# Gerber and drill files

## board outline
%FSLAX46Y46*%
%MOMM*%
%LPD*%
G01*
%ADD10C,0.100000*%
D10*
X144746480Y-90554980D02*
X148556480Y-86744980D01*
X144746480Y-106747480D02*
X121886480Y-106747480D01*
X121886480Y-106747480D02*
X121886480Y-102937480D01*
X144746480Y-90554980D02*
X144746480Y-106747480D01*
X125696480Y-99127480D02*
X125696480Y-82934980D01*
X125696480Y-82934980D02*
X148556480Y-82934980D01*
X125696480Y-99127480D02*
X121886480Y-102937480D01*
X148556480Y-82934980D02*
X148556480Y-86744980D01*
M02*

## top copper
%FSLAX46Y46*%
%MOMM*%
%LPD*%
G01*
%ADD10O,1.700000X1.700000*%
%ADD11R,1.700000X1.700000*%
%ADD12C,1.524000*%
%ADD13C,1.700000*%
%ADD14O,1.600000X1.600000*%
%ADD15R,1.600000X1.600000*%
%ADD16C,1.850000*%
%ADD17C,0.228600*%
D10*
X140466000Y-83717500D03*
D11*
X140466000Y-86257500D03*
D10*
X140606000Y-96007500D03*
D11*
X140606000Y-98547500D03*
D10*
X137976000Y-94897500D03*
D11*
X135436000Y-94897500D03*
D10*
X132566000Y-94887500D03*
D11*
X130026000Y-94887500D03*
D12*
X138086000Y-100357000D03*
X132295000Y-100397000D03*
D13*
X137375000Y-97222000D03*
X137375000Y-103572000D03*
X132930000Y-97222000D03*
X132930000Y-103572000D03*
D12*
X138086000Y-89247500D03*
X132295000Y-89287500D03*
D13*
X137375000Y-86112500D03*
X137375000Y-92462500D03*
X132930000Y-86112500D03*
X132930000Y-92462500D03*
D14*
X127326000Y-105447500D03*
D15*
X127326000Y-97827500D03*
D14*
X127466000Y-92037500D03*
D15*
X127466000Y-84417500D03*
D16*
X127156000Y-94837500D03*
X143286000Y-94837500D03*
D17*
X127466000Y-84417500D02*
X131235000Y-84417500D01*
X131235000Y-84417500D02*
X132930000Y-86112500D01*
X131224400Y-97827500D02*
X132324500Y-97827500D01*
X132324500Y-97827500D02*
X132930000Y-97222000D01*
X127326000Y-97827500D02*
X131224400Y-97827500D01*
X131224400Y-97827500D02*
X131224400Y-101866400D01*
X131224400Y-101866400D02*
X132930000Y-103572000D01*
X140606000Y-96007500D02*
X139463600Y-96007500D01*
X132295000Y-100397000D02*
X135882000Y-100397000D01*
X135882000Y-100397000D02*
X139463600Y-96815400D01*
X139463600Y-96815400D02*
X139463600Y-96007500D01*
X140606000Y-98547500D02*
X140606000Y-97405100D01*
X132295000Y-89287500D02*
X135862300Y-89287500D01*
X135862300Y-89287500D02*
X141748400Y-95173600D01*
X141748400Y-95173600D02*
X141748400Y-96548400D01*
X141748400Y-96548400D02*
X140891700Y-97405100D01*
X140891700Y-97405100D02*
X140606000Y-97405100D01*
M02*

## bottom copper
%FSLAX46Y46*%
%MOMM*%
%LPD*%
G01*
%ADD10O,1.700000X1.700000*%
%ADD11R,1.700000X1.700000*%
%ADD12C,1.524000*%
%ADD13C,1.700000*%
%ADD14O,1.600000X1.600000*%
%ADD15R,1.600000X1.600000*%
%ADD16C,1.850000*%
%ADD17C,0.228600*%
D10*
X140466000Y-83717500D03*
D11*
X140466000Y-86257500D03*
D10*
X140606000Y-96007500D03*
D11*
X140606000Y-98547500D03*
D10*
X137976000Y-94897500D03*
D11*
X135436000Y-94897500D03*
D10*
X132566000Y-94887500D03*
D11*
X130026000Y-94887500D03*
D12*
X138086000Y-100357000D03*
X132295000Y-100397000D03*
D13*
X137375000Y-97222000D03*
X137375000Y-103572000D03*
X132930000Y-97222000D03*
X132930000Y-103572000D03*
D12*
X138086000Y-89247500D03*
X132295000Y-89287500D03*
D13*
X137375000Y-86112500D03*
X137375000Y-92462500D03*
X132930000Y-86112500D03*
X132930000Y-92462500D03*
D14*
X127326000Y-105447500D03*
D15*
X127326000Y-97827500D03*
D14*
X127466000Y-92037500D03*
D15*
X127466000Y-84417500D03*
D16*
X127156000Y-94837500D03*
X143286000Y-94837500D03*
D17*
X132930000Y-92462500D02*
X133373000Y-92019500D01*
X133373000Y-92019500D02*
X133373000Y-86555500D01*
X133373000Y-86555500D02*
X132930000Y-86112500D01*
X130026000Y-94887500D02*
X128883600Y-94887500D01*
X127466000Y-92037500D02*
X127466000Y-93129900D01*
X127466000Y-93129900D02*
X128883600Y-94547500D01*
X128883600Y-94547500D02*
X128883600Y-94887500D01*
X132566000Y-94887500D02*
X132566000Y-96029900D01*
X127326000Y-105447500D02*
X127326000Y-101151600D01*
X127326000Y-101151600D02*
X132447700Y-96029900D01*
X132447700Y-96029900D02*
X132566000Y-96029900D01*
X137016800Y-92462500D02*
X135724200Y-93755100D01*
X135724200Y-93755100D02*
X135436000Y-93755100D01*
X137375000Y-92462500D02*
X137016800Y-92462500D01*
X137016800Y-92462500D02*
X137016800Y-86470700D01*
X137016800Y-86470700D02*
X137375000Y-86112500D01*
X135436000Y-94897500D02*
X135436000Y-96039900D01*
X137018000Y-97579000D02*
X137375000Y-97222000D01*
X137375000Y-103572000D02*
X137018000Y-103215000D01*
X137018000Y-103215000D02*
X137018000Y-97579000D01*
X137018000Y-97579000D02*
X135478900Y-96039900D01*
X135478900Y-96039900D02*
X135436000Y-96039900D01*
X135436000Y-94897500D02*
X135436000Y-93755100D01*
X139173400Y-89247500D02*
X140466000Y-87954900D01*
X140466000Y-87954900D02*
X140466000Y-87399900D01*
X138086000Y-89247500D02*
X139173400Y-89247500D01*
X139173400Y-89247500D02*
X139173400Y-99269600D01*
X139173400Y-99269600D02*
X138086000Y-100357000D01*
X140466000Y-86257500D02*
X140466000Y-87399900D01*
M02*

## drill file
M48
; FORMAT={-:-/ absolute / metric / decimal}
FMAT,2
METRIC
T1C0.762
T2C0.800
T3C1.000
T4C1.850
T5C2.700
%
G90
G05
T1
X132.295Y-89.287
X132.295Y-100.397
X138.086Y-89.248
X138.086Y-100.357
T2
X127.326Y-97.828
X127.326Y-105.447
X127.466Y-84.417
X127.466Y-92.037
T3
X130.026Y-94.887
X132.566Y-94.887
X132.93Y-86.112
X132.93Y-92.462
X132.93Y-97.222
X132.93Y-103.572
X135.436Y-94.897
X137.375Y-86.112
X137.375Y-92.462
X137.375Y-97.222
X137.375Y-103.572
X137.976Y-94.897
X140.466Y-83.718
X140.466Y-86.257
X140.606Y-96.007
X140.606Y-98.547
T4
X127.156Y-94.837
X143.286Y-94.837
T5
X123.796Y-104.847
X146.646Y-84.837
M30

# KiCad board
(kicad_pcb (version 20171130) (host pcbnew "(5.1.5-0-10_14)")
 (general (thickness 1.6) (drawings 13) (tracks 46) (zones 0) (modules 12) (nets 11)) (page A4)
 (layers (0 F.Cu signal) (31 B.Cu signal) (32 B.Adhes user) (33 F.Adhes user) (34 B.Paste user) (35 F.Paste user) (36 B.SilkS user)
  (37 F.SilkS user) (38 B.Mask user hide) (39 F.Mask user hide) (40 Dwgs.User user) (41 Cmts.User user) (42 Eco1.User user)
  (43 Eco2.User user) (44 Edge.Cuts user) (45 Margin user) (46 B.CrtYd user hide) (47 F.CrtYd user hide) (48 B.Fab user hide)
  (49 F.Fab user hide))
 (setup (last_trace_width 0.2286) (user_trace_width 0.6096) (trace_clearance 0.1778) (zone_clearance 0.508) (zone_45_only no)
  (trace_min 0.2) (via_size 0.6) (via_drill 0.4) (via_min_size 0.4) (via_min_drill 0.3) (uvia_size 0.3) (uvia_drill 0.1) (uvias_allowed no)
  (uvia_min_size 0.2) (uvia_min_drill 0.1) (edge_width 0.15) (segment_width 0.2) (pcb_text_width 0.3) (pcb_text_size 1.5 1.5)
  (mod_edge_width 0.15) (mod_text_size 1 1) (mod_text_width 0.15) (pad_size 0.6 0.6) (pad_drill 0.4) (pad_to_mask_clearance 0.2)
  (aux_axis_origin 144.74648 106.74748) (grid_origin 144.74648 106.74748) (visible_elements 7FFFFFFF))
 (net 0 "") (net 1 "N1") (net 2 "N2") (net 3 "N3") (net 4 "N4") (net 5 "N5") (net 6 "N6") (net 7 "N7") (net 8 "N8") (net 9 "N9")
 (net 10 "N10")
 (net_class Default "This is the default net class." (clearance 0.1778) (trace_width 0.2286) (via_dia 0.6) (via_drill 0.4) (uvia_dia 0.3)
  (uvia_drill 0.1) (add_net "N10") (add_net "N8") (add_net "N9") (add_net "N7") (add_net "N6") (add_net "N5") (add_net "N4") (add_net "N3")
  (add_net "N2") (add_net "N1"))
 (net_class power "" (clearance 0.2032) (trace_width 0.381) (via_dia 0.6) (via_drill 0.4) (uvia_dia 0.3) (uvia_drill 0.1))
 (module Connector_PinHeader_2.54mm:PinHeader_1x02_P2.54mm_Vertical (layer B.Cu) (at 140.466 86.2575)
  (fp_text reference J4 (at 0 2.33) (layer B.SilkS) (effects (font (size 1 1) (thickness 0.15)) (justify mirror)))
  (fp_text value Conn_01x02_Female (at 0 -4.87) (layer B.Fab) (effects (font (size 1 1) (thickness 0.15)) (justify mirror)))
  (pad 2 thru_hole oval (at 0 -2.54) (size 1.7 1.7) (drill 1) (layers *.Cu *.Mask) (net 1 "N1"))
  (pad 1 thru_hole rect (at 0 0) (size 1.7 1.7) (drill 1) (layers *.Cu *.Mask) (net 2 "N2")))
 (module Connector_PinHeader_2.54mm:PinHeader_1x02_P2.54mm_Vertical (layer B.Cu) (at 140.606 98.5475)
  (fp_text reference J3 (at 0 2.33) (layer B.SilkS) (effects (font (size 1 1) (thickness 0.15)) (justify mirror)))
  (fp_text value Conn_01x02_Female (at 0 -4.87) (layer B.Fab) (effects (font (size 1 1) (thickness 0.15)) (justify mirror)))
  (pad 2 thru_hole oval (at 0 -2.54) (size 1.7 1.7) (drill 1) (layers *.Cu *.Mask) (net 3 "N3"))
  (pad 1 thru_hole rect (at 0 0) (size 1.7 1.7) (drill 1) (layers *.Cu *.Mask) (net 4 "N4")))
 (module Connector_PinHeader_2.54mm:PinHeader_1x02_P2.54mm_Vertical (layer B.Cu) (at 135.436 94.8975 270)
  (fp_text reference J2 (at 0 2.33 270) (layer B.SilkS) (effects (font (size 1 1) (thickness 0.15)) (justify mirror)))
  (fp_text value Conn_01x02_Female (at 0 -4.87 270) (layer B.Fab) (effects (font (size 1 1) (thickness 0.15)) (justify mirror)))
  (pad 2 thru_hole oval (at 0 -2.54 270) (size 1.7 1.7) (drill 1) (layers *.Cu *.Mask) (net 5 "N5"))
  (pad 1 thru_hole rect (at 0 0 270) (size 1.7 1.7) (drill 1) (layers *.Cu *.Mask) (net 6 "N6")))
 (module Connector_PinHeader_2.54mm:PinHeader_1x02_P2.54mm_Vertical (layer B.Cu) (at 130.026 94.8875 270)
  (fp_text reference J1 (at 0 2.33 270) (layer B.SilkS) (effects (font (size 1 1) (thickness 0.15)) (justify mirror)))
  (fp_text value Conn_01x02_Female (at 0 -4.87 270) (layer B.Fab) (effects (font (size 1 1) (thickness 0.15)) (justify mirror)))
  (pad 2 thru_hole oval (at 0 -2.54 270) (size 1.7 1.7) (drill 1) (layers *.Cu *.Mask) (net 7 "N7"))
  (pad 1 thru_hole rect (at 0 0 270) (size 1.7 1.7) (drill 1) (layers *.Cu *.Mask) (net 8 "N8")))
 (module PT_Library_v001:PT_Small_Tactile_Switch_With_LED (layer F.Cu) (at 135.216 100.397 90)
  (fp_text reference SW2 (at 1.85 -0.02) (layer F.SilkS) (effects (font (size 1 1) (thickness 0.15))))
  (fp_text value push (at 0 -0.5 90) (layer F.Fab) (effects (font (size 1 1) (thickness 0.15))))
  (pad 6 thru_hole circle (at 0.04 2.87 90) (size 1.524 1.524) (drill 0.762) (layers *.Cu *.Mask) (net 2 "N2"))
  (pad 5 thru_hole circle (at 0 -2.921 90) (size 1.524 1.524) (drill 0.762) (layers *.Cu *.Mask) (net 3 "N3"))
  (pad 4 thru_hole circle (at 3.175 2.159 90) (size 1.7 1.7) (drill 1) (layers *.Cu *.Mask) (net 6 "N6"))
  (pad 3 thru_hole circle (at -3.175 2.159 90) (size 1.7 1.7) (drill 1) (layers *.Cu *.Mask) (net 6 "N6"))
  (pad 2 thru_hole circle (at 3.175 -2.286 90) (size 1.7 1.7) (drill 1) (layers *.Cu *.Mask) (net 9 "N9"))
  (pad 1 thru_hole circle (at -3.175 -2.286 90) (size 1.7 1.7) (drill 1) (layers *.Cu *.Mask) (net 9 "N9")))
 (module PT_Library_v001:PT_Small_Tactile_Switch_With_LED (layer F.Cu) (at 135.216 89.2875 90)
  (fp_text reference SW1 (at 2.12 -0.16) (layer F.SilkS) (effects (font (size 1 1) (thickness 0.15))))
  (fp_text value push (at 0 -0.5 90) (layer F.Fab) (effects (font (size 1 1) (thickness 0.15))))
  (pad 6 thru_hole circle (at 0.04 2.87 90) (size 1.524 1.524) (drill 0.762) (layers *.Cu *.Mask) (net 2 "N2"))
  (pad 5 thru_hole circle (at 0 -2.921 90) (size 1.524 1.524) (drill 0.762) (layers *.Cu *.Mask) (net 4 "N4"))
  (pad 4 thru_hole circle (at 3.175 2.159 90) (size 1.7 1.7) (drill 1) (layers *.Cu *.Mask) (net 6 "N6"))
  (pad 3 thru_hole circle (at -3.175 2.159 90) (size 1.7 1.7) (drill 1) (layers *.Cu *.Mask) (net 6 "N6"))
  (pad 2 thru_hole circle (at 3.175 -2.286 90) (size 1.7 1.7) (drill 1) (layers *.Cu *.Mask) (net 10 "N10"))
  (pad 1 thru_hole circle (at -3.175 -2.286 90) (size 1.7 1.7) (drill 1) (layers *.Cu *.Mask) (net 10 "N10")))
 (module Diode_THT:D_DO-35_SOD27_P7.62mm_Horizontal (layer F.Cu) (at 127.326 97.8275 270)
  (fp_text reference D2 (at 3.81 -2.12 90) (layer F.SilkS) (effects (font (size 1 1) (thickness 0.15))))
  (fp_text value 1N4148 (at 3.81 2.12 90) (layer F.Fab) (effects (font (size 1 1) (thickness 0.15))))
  (pad 2 thru_hole oval (at 7.62 0 270) (size 1.6 1.6) (drill 0.8) (layers *.Cu *.Mask) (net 7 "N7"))
  (pad 1 thru_hole rect (at 0 0 270) (size 1.6 1.6) (drill 0.8) (layers *.Cu *.Mask) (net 9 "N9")))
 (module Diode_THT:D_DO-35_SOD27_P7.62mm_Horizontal (layer F.Cu) (at 127.466 84.4175 270)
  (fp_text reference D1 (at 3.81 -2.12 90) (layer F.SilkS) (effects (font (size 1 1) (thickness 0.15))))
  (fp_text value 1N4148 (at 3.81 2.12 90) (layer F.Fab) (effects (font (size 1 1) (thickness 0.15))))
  (pad 2 thru_hole oval (at 7.62 0 270) (size 1.6 1.6) (drill 0.8) (layers *.Cu *.Mask) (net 8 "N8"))
  (pad 1 thru_hole rect (at 0 0 270) (size 1.6 1.6) (drill 0.8) (layers *.Cu *.Mask) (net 10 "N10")))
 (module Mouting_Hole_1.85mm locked (layer F.Cu) (at 127.156 94.8375 180)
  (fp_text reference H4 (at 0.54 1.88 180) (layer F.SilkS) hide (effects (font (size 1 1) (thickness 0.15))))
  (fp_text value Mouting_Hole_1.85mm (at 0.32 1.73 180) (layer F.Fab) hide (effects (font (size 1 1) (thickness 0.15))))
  (pad 1 thru_hole circle (at 0 0 180) (size 1.85 1.85) (drill 1.85) (layers *.Cu) (clearance 0.5) (zone_connect 0)))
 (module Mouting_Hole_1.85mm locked (layer F.Cu) (at 143.286 94.8375 180)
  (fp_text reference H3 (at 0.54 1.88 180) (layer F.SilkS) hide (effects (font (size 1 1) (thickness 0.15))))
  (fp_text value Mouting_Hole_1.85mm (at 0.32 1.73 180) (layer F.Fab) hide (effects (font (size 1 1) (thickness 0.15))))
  (pad 1 thru_hole circle (at 0 0 180) (size 1.85 1.85) (drill 1.85) (layers *.Cu) (clearance 0.5) (zone_connect 0)))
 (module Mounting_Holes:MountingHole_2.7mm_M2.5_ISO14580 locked (layer F.Cu) (at 146.646 84.8375 180)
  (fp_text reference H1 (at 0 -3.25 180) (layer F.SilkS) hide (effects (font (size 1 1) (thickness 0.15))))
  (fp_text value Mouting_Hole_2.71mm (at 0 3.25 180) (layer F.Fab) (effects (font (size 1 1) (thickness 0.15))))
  (pad 1 np_thru_hole circle (at 0 0 180) (size 2.7 2.7) (drill 2.7) (layers *.Cu *.Mask)))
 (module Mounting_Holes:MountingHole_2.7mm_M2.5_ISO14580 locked (layer F.Cu) (at 123.796 104.847 180)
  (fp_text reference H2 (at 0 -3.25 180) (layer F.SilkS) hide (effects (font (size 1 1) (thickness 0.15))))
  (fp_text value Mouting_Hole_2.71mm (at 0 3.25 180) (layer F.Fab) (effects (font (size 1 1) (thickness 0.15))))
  (pad 1 np_thru_hole circle (at 0 0 180) (size 2.7 2.7) (drill 2.7) (layers *.Cu *.Mask)))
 (gr_line (start 144.74648 90.55498) (end 148.55648 86.74498) (layer Edge.Cuts) (width 0.1))
 (gr_line (start 144.74648 106.74748) (end 121.88648 106.74748) (layer Edge.Cuts) (width 0.1))
 (gr_line (start 121.88648 106.74748) (end 121.88648 102.93748) (layer Edge.Cuts) (width 0.1))
 (gr_line (start 144.74648 90.55498) (end 144.74648 106.74748) (layer Edge.Cuts) (width 0.1))
 (gr_line (start 125.69648 99.12748) (end 125.69648 82.93498) (layer Edge.Cuts) (width 0.1))
 (gr_line (start 125.69648 82.93498) (end 148.55648 82.93498) (layer Edge.Cuts) (width 0.1))
 (gr_line (start 125.69648 99.12748) (end 121.88648 102.93748) (layer Edge.Cuts) (width 0.1))
 (gr_line (start 148.55648 82.93498) (end 148.55648 86.74498) (layer Edge.Cuts) (width 0.1))
 (segment (start 132.93 92.4625) (end 133.373 92.0195) (width 0.2286) (layer B.Cu) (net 10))
 (segment (start 133.373 92.0195) (end 133.373 86.5555) (width 0.2286) (layer B.Cu) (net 10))
 (segment (start 133.373 86.5555) (end 132.93 86.1125) (width 0.2286) (layer B.Cu) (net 10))
 (segment (start 127.466 84.4175) (end 131.235 84.4175) (width 0.2286) (layer F.Cu) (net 10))
 (segment (start 131.235 84.4175) (end 132.93 86.1125) (width 0.2286) (layer F.Cu) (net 10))
 (segment (start 130.026 94.8875) (end 128.8836 94.8875) (width 0.2286) (layer B.Cu) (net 8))
 (segment (start 127.466 92.0375) (end 127.466 93.1299) (width 0.2286) (layer B.Cu) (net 8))
 (segment (start 127.466 93.1299) (end 128.8836 94.5475) (width 0.2286) (layer B.Cu) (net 8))
 (segment (start 128.8836 94.5475) (end 128.8836 94.8875) (width 0.2286) (layer B.Cu) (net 8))
 (segment (start 132.566 94.8875) (end 132.566 96.0299) (width 0.2286) (layer B.Cu) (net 7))
 (segment (start 127.326 105.4475) (end 127.326 101.1516) (width 0.2286) (layer B.Cu) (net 7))
 (segment (start 127.326 101.1516) (end 132.4477 96.0299) (width 0.2286) (layer B.Cu) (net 7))
 (segment (start 132.4477 96.0299) (end 132.566 96.0299) (width 0.2286) (layer B.Cu) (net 7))
 (segment (start 131.2244 97.8275) (end 132.3245 97.8275) (width 0.2286) (layer F.Cu) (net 9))
 (segment (start 132.3245 97.8275) (end 132.93 97.222) (width 0.2286) (layer F.Cu) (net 9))
 (segment (start 127.326 97.8275) (end 131.2244 97.8275) (width 0.2286) (layer F.Cu) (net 9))
 (segment (start 131.2244 97.8275) (end 131.2244 101.8664) (width 0.2286) (layer F.Cu) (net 9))
 (segment (start 131.2244 101.8664) (end 132.93 103.572) (width 0.2286) (layer F.Cu) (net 9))
 (segment (start 137.0168 92.4625) (end 135.7242 93.7551) (width 0.2286) (layer B.Cu) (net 6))
 (segment (start 135.7242 93.7551) (end 135.436 93.7551) (width 0.2286) (layer B.Cu) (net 6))
 (segment (start 137.375 92.4625) (end 137.0168 92.4625) (width 0.2286) (layer B.Cu) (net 6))
 (segment (start 137.0168 92.4625) (end 137.0168 86.4707) (width 0.2286) (layer B.Cu) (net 6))
 (segment (start 137.0168 86.4707) (end 137.375 86.1125) (width 0.2286) (layer B.Cu) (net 6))
 (segment (start 135.436 94.8975) (end 135.436 96.0399) (width 0.2286) (layer B.Cu) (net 6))
 (segment (start 137.018 97.579) (end 137.375 97.222) (width 0.2286) (layer B.Cu) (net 6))
 (segment (start 137.375 103.572) (end 137.018 103.215) (width 0.2286) (layer B.Cu) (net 6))
 (segment (start 137.018 103.215) (end 137.018 97.579) (width 0.2286) (layer B.Cu) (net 6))
 (segment (start 137.018 97.579) (end 135.4789 96.0399) (width 0.2286) (layer B.Cu) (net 6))
 (segment (start 135.4789 96.0399) (end 135.436 96.0399) (width 0.2286) (layer B.Cu) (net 6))
 (segment (start 135.436 94.8975) (end 135.436 93.7551) (width 0.2286) (layer B.Cu) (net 6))
 (segment (start 140.606 96.0075) (end 139.4636 96.0075) (width 0.2286) (layer F.Cu) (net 3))
 (segment (start 132.295 100.397) (end 135.882 100.397) (width 0.2286) (layer F.Cu) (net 3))
 (segment (start 135.882 100.397) (end 139.4636 96.8154) (width 0.2286) (layer F.Cu) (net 3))
 (segment (start 139.4636 96.8154) (end 139.4636 96.0075) (width 0.2286) (layer F.Cu) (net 3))
 (segment (start 140.606 98.5475) (end 140.606 97.4051) (width 0.2286) (layer F.Cu) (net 4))
 (segment (start 132.295 89.2875) (end 135.8623 89.2875) (width 0.2286) (layer F.Cu) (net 4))
 (segment (start 135.8623 89.2875) (end 141.7484 95.1736) (width 0.2286) (layer F.Cu) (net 4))
 (segment (start 141.7484 95.1736) (end 141.7484 96.5484) (width 0.2286) (layer F.Cu) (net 4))
 (segment (start 141.7484 96.5484) (end 140.8917 97.4051) (width 0.2286) (layer F.Cu) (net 4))
 (segment (start 140.8917 97.4051) (end 140.606 97.4051) (width 0.2286) (layer F.Cu) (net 4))
 (segment (start 139.1734 89.2475) (end 140.466 87.9549) (width 0.2286) (layer B.Cu) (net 2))
 (segment (start 140.466 87.9549) (end 140.466 87.3999) (width 0.2286) (layer B.Cu) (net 2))
 (segment (start 138.086 89.2475) (end 139.1734 89.2475) (width 0.2286) (layer B.Cu) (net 2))
 (segment (start 139.1734 89.2475) (end 139.1734 99.2696) (width 0.2286) (layer B.Cu) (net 2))
 (segment (start 139.1734 99.2696) (end 138.086 100.357) (width 0.2286) (layer B.Cu) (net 2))
 (segment (start 140.466 86.2575) (end 140.466 87.3999) (width 0.2286) (layer B.Cu) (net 2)))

